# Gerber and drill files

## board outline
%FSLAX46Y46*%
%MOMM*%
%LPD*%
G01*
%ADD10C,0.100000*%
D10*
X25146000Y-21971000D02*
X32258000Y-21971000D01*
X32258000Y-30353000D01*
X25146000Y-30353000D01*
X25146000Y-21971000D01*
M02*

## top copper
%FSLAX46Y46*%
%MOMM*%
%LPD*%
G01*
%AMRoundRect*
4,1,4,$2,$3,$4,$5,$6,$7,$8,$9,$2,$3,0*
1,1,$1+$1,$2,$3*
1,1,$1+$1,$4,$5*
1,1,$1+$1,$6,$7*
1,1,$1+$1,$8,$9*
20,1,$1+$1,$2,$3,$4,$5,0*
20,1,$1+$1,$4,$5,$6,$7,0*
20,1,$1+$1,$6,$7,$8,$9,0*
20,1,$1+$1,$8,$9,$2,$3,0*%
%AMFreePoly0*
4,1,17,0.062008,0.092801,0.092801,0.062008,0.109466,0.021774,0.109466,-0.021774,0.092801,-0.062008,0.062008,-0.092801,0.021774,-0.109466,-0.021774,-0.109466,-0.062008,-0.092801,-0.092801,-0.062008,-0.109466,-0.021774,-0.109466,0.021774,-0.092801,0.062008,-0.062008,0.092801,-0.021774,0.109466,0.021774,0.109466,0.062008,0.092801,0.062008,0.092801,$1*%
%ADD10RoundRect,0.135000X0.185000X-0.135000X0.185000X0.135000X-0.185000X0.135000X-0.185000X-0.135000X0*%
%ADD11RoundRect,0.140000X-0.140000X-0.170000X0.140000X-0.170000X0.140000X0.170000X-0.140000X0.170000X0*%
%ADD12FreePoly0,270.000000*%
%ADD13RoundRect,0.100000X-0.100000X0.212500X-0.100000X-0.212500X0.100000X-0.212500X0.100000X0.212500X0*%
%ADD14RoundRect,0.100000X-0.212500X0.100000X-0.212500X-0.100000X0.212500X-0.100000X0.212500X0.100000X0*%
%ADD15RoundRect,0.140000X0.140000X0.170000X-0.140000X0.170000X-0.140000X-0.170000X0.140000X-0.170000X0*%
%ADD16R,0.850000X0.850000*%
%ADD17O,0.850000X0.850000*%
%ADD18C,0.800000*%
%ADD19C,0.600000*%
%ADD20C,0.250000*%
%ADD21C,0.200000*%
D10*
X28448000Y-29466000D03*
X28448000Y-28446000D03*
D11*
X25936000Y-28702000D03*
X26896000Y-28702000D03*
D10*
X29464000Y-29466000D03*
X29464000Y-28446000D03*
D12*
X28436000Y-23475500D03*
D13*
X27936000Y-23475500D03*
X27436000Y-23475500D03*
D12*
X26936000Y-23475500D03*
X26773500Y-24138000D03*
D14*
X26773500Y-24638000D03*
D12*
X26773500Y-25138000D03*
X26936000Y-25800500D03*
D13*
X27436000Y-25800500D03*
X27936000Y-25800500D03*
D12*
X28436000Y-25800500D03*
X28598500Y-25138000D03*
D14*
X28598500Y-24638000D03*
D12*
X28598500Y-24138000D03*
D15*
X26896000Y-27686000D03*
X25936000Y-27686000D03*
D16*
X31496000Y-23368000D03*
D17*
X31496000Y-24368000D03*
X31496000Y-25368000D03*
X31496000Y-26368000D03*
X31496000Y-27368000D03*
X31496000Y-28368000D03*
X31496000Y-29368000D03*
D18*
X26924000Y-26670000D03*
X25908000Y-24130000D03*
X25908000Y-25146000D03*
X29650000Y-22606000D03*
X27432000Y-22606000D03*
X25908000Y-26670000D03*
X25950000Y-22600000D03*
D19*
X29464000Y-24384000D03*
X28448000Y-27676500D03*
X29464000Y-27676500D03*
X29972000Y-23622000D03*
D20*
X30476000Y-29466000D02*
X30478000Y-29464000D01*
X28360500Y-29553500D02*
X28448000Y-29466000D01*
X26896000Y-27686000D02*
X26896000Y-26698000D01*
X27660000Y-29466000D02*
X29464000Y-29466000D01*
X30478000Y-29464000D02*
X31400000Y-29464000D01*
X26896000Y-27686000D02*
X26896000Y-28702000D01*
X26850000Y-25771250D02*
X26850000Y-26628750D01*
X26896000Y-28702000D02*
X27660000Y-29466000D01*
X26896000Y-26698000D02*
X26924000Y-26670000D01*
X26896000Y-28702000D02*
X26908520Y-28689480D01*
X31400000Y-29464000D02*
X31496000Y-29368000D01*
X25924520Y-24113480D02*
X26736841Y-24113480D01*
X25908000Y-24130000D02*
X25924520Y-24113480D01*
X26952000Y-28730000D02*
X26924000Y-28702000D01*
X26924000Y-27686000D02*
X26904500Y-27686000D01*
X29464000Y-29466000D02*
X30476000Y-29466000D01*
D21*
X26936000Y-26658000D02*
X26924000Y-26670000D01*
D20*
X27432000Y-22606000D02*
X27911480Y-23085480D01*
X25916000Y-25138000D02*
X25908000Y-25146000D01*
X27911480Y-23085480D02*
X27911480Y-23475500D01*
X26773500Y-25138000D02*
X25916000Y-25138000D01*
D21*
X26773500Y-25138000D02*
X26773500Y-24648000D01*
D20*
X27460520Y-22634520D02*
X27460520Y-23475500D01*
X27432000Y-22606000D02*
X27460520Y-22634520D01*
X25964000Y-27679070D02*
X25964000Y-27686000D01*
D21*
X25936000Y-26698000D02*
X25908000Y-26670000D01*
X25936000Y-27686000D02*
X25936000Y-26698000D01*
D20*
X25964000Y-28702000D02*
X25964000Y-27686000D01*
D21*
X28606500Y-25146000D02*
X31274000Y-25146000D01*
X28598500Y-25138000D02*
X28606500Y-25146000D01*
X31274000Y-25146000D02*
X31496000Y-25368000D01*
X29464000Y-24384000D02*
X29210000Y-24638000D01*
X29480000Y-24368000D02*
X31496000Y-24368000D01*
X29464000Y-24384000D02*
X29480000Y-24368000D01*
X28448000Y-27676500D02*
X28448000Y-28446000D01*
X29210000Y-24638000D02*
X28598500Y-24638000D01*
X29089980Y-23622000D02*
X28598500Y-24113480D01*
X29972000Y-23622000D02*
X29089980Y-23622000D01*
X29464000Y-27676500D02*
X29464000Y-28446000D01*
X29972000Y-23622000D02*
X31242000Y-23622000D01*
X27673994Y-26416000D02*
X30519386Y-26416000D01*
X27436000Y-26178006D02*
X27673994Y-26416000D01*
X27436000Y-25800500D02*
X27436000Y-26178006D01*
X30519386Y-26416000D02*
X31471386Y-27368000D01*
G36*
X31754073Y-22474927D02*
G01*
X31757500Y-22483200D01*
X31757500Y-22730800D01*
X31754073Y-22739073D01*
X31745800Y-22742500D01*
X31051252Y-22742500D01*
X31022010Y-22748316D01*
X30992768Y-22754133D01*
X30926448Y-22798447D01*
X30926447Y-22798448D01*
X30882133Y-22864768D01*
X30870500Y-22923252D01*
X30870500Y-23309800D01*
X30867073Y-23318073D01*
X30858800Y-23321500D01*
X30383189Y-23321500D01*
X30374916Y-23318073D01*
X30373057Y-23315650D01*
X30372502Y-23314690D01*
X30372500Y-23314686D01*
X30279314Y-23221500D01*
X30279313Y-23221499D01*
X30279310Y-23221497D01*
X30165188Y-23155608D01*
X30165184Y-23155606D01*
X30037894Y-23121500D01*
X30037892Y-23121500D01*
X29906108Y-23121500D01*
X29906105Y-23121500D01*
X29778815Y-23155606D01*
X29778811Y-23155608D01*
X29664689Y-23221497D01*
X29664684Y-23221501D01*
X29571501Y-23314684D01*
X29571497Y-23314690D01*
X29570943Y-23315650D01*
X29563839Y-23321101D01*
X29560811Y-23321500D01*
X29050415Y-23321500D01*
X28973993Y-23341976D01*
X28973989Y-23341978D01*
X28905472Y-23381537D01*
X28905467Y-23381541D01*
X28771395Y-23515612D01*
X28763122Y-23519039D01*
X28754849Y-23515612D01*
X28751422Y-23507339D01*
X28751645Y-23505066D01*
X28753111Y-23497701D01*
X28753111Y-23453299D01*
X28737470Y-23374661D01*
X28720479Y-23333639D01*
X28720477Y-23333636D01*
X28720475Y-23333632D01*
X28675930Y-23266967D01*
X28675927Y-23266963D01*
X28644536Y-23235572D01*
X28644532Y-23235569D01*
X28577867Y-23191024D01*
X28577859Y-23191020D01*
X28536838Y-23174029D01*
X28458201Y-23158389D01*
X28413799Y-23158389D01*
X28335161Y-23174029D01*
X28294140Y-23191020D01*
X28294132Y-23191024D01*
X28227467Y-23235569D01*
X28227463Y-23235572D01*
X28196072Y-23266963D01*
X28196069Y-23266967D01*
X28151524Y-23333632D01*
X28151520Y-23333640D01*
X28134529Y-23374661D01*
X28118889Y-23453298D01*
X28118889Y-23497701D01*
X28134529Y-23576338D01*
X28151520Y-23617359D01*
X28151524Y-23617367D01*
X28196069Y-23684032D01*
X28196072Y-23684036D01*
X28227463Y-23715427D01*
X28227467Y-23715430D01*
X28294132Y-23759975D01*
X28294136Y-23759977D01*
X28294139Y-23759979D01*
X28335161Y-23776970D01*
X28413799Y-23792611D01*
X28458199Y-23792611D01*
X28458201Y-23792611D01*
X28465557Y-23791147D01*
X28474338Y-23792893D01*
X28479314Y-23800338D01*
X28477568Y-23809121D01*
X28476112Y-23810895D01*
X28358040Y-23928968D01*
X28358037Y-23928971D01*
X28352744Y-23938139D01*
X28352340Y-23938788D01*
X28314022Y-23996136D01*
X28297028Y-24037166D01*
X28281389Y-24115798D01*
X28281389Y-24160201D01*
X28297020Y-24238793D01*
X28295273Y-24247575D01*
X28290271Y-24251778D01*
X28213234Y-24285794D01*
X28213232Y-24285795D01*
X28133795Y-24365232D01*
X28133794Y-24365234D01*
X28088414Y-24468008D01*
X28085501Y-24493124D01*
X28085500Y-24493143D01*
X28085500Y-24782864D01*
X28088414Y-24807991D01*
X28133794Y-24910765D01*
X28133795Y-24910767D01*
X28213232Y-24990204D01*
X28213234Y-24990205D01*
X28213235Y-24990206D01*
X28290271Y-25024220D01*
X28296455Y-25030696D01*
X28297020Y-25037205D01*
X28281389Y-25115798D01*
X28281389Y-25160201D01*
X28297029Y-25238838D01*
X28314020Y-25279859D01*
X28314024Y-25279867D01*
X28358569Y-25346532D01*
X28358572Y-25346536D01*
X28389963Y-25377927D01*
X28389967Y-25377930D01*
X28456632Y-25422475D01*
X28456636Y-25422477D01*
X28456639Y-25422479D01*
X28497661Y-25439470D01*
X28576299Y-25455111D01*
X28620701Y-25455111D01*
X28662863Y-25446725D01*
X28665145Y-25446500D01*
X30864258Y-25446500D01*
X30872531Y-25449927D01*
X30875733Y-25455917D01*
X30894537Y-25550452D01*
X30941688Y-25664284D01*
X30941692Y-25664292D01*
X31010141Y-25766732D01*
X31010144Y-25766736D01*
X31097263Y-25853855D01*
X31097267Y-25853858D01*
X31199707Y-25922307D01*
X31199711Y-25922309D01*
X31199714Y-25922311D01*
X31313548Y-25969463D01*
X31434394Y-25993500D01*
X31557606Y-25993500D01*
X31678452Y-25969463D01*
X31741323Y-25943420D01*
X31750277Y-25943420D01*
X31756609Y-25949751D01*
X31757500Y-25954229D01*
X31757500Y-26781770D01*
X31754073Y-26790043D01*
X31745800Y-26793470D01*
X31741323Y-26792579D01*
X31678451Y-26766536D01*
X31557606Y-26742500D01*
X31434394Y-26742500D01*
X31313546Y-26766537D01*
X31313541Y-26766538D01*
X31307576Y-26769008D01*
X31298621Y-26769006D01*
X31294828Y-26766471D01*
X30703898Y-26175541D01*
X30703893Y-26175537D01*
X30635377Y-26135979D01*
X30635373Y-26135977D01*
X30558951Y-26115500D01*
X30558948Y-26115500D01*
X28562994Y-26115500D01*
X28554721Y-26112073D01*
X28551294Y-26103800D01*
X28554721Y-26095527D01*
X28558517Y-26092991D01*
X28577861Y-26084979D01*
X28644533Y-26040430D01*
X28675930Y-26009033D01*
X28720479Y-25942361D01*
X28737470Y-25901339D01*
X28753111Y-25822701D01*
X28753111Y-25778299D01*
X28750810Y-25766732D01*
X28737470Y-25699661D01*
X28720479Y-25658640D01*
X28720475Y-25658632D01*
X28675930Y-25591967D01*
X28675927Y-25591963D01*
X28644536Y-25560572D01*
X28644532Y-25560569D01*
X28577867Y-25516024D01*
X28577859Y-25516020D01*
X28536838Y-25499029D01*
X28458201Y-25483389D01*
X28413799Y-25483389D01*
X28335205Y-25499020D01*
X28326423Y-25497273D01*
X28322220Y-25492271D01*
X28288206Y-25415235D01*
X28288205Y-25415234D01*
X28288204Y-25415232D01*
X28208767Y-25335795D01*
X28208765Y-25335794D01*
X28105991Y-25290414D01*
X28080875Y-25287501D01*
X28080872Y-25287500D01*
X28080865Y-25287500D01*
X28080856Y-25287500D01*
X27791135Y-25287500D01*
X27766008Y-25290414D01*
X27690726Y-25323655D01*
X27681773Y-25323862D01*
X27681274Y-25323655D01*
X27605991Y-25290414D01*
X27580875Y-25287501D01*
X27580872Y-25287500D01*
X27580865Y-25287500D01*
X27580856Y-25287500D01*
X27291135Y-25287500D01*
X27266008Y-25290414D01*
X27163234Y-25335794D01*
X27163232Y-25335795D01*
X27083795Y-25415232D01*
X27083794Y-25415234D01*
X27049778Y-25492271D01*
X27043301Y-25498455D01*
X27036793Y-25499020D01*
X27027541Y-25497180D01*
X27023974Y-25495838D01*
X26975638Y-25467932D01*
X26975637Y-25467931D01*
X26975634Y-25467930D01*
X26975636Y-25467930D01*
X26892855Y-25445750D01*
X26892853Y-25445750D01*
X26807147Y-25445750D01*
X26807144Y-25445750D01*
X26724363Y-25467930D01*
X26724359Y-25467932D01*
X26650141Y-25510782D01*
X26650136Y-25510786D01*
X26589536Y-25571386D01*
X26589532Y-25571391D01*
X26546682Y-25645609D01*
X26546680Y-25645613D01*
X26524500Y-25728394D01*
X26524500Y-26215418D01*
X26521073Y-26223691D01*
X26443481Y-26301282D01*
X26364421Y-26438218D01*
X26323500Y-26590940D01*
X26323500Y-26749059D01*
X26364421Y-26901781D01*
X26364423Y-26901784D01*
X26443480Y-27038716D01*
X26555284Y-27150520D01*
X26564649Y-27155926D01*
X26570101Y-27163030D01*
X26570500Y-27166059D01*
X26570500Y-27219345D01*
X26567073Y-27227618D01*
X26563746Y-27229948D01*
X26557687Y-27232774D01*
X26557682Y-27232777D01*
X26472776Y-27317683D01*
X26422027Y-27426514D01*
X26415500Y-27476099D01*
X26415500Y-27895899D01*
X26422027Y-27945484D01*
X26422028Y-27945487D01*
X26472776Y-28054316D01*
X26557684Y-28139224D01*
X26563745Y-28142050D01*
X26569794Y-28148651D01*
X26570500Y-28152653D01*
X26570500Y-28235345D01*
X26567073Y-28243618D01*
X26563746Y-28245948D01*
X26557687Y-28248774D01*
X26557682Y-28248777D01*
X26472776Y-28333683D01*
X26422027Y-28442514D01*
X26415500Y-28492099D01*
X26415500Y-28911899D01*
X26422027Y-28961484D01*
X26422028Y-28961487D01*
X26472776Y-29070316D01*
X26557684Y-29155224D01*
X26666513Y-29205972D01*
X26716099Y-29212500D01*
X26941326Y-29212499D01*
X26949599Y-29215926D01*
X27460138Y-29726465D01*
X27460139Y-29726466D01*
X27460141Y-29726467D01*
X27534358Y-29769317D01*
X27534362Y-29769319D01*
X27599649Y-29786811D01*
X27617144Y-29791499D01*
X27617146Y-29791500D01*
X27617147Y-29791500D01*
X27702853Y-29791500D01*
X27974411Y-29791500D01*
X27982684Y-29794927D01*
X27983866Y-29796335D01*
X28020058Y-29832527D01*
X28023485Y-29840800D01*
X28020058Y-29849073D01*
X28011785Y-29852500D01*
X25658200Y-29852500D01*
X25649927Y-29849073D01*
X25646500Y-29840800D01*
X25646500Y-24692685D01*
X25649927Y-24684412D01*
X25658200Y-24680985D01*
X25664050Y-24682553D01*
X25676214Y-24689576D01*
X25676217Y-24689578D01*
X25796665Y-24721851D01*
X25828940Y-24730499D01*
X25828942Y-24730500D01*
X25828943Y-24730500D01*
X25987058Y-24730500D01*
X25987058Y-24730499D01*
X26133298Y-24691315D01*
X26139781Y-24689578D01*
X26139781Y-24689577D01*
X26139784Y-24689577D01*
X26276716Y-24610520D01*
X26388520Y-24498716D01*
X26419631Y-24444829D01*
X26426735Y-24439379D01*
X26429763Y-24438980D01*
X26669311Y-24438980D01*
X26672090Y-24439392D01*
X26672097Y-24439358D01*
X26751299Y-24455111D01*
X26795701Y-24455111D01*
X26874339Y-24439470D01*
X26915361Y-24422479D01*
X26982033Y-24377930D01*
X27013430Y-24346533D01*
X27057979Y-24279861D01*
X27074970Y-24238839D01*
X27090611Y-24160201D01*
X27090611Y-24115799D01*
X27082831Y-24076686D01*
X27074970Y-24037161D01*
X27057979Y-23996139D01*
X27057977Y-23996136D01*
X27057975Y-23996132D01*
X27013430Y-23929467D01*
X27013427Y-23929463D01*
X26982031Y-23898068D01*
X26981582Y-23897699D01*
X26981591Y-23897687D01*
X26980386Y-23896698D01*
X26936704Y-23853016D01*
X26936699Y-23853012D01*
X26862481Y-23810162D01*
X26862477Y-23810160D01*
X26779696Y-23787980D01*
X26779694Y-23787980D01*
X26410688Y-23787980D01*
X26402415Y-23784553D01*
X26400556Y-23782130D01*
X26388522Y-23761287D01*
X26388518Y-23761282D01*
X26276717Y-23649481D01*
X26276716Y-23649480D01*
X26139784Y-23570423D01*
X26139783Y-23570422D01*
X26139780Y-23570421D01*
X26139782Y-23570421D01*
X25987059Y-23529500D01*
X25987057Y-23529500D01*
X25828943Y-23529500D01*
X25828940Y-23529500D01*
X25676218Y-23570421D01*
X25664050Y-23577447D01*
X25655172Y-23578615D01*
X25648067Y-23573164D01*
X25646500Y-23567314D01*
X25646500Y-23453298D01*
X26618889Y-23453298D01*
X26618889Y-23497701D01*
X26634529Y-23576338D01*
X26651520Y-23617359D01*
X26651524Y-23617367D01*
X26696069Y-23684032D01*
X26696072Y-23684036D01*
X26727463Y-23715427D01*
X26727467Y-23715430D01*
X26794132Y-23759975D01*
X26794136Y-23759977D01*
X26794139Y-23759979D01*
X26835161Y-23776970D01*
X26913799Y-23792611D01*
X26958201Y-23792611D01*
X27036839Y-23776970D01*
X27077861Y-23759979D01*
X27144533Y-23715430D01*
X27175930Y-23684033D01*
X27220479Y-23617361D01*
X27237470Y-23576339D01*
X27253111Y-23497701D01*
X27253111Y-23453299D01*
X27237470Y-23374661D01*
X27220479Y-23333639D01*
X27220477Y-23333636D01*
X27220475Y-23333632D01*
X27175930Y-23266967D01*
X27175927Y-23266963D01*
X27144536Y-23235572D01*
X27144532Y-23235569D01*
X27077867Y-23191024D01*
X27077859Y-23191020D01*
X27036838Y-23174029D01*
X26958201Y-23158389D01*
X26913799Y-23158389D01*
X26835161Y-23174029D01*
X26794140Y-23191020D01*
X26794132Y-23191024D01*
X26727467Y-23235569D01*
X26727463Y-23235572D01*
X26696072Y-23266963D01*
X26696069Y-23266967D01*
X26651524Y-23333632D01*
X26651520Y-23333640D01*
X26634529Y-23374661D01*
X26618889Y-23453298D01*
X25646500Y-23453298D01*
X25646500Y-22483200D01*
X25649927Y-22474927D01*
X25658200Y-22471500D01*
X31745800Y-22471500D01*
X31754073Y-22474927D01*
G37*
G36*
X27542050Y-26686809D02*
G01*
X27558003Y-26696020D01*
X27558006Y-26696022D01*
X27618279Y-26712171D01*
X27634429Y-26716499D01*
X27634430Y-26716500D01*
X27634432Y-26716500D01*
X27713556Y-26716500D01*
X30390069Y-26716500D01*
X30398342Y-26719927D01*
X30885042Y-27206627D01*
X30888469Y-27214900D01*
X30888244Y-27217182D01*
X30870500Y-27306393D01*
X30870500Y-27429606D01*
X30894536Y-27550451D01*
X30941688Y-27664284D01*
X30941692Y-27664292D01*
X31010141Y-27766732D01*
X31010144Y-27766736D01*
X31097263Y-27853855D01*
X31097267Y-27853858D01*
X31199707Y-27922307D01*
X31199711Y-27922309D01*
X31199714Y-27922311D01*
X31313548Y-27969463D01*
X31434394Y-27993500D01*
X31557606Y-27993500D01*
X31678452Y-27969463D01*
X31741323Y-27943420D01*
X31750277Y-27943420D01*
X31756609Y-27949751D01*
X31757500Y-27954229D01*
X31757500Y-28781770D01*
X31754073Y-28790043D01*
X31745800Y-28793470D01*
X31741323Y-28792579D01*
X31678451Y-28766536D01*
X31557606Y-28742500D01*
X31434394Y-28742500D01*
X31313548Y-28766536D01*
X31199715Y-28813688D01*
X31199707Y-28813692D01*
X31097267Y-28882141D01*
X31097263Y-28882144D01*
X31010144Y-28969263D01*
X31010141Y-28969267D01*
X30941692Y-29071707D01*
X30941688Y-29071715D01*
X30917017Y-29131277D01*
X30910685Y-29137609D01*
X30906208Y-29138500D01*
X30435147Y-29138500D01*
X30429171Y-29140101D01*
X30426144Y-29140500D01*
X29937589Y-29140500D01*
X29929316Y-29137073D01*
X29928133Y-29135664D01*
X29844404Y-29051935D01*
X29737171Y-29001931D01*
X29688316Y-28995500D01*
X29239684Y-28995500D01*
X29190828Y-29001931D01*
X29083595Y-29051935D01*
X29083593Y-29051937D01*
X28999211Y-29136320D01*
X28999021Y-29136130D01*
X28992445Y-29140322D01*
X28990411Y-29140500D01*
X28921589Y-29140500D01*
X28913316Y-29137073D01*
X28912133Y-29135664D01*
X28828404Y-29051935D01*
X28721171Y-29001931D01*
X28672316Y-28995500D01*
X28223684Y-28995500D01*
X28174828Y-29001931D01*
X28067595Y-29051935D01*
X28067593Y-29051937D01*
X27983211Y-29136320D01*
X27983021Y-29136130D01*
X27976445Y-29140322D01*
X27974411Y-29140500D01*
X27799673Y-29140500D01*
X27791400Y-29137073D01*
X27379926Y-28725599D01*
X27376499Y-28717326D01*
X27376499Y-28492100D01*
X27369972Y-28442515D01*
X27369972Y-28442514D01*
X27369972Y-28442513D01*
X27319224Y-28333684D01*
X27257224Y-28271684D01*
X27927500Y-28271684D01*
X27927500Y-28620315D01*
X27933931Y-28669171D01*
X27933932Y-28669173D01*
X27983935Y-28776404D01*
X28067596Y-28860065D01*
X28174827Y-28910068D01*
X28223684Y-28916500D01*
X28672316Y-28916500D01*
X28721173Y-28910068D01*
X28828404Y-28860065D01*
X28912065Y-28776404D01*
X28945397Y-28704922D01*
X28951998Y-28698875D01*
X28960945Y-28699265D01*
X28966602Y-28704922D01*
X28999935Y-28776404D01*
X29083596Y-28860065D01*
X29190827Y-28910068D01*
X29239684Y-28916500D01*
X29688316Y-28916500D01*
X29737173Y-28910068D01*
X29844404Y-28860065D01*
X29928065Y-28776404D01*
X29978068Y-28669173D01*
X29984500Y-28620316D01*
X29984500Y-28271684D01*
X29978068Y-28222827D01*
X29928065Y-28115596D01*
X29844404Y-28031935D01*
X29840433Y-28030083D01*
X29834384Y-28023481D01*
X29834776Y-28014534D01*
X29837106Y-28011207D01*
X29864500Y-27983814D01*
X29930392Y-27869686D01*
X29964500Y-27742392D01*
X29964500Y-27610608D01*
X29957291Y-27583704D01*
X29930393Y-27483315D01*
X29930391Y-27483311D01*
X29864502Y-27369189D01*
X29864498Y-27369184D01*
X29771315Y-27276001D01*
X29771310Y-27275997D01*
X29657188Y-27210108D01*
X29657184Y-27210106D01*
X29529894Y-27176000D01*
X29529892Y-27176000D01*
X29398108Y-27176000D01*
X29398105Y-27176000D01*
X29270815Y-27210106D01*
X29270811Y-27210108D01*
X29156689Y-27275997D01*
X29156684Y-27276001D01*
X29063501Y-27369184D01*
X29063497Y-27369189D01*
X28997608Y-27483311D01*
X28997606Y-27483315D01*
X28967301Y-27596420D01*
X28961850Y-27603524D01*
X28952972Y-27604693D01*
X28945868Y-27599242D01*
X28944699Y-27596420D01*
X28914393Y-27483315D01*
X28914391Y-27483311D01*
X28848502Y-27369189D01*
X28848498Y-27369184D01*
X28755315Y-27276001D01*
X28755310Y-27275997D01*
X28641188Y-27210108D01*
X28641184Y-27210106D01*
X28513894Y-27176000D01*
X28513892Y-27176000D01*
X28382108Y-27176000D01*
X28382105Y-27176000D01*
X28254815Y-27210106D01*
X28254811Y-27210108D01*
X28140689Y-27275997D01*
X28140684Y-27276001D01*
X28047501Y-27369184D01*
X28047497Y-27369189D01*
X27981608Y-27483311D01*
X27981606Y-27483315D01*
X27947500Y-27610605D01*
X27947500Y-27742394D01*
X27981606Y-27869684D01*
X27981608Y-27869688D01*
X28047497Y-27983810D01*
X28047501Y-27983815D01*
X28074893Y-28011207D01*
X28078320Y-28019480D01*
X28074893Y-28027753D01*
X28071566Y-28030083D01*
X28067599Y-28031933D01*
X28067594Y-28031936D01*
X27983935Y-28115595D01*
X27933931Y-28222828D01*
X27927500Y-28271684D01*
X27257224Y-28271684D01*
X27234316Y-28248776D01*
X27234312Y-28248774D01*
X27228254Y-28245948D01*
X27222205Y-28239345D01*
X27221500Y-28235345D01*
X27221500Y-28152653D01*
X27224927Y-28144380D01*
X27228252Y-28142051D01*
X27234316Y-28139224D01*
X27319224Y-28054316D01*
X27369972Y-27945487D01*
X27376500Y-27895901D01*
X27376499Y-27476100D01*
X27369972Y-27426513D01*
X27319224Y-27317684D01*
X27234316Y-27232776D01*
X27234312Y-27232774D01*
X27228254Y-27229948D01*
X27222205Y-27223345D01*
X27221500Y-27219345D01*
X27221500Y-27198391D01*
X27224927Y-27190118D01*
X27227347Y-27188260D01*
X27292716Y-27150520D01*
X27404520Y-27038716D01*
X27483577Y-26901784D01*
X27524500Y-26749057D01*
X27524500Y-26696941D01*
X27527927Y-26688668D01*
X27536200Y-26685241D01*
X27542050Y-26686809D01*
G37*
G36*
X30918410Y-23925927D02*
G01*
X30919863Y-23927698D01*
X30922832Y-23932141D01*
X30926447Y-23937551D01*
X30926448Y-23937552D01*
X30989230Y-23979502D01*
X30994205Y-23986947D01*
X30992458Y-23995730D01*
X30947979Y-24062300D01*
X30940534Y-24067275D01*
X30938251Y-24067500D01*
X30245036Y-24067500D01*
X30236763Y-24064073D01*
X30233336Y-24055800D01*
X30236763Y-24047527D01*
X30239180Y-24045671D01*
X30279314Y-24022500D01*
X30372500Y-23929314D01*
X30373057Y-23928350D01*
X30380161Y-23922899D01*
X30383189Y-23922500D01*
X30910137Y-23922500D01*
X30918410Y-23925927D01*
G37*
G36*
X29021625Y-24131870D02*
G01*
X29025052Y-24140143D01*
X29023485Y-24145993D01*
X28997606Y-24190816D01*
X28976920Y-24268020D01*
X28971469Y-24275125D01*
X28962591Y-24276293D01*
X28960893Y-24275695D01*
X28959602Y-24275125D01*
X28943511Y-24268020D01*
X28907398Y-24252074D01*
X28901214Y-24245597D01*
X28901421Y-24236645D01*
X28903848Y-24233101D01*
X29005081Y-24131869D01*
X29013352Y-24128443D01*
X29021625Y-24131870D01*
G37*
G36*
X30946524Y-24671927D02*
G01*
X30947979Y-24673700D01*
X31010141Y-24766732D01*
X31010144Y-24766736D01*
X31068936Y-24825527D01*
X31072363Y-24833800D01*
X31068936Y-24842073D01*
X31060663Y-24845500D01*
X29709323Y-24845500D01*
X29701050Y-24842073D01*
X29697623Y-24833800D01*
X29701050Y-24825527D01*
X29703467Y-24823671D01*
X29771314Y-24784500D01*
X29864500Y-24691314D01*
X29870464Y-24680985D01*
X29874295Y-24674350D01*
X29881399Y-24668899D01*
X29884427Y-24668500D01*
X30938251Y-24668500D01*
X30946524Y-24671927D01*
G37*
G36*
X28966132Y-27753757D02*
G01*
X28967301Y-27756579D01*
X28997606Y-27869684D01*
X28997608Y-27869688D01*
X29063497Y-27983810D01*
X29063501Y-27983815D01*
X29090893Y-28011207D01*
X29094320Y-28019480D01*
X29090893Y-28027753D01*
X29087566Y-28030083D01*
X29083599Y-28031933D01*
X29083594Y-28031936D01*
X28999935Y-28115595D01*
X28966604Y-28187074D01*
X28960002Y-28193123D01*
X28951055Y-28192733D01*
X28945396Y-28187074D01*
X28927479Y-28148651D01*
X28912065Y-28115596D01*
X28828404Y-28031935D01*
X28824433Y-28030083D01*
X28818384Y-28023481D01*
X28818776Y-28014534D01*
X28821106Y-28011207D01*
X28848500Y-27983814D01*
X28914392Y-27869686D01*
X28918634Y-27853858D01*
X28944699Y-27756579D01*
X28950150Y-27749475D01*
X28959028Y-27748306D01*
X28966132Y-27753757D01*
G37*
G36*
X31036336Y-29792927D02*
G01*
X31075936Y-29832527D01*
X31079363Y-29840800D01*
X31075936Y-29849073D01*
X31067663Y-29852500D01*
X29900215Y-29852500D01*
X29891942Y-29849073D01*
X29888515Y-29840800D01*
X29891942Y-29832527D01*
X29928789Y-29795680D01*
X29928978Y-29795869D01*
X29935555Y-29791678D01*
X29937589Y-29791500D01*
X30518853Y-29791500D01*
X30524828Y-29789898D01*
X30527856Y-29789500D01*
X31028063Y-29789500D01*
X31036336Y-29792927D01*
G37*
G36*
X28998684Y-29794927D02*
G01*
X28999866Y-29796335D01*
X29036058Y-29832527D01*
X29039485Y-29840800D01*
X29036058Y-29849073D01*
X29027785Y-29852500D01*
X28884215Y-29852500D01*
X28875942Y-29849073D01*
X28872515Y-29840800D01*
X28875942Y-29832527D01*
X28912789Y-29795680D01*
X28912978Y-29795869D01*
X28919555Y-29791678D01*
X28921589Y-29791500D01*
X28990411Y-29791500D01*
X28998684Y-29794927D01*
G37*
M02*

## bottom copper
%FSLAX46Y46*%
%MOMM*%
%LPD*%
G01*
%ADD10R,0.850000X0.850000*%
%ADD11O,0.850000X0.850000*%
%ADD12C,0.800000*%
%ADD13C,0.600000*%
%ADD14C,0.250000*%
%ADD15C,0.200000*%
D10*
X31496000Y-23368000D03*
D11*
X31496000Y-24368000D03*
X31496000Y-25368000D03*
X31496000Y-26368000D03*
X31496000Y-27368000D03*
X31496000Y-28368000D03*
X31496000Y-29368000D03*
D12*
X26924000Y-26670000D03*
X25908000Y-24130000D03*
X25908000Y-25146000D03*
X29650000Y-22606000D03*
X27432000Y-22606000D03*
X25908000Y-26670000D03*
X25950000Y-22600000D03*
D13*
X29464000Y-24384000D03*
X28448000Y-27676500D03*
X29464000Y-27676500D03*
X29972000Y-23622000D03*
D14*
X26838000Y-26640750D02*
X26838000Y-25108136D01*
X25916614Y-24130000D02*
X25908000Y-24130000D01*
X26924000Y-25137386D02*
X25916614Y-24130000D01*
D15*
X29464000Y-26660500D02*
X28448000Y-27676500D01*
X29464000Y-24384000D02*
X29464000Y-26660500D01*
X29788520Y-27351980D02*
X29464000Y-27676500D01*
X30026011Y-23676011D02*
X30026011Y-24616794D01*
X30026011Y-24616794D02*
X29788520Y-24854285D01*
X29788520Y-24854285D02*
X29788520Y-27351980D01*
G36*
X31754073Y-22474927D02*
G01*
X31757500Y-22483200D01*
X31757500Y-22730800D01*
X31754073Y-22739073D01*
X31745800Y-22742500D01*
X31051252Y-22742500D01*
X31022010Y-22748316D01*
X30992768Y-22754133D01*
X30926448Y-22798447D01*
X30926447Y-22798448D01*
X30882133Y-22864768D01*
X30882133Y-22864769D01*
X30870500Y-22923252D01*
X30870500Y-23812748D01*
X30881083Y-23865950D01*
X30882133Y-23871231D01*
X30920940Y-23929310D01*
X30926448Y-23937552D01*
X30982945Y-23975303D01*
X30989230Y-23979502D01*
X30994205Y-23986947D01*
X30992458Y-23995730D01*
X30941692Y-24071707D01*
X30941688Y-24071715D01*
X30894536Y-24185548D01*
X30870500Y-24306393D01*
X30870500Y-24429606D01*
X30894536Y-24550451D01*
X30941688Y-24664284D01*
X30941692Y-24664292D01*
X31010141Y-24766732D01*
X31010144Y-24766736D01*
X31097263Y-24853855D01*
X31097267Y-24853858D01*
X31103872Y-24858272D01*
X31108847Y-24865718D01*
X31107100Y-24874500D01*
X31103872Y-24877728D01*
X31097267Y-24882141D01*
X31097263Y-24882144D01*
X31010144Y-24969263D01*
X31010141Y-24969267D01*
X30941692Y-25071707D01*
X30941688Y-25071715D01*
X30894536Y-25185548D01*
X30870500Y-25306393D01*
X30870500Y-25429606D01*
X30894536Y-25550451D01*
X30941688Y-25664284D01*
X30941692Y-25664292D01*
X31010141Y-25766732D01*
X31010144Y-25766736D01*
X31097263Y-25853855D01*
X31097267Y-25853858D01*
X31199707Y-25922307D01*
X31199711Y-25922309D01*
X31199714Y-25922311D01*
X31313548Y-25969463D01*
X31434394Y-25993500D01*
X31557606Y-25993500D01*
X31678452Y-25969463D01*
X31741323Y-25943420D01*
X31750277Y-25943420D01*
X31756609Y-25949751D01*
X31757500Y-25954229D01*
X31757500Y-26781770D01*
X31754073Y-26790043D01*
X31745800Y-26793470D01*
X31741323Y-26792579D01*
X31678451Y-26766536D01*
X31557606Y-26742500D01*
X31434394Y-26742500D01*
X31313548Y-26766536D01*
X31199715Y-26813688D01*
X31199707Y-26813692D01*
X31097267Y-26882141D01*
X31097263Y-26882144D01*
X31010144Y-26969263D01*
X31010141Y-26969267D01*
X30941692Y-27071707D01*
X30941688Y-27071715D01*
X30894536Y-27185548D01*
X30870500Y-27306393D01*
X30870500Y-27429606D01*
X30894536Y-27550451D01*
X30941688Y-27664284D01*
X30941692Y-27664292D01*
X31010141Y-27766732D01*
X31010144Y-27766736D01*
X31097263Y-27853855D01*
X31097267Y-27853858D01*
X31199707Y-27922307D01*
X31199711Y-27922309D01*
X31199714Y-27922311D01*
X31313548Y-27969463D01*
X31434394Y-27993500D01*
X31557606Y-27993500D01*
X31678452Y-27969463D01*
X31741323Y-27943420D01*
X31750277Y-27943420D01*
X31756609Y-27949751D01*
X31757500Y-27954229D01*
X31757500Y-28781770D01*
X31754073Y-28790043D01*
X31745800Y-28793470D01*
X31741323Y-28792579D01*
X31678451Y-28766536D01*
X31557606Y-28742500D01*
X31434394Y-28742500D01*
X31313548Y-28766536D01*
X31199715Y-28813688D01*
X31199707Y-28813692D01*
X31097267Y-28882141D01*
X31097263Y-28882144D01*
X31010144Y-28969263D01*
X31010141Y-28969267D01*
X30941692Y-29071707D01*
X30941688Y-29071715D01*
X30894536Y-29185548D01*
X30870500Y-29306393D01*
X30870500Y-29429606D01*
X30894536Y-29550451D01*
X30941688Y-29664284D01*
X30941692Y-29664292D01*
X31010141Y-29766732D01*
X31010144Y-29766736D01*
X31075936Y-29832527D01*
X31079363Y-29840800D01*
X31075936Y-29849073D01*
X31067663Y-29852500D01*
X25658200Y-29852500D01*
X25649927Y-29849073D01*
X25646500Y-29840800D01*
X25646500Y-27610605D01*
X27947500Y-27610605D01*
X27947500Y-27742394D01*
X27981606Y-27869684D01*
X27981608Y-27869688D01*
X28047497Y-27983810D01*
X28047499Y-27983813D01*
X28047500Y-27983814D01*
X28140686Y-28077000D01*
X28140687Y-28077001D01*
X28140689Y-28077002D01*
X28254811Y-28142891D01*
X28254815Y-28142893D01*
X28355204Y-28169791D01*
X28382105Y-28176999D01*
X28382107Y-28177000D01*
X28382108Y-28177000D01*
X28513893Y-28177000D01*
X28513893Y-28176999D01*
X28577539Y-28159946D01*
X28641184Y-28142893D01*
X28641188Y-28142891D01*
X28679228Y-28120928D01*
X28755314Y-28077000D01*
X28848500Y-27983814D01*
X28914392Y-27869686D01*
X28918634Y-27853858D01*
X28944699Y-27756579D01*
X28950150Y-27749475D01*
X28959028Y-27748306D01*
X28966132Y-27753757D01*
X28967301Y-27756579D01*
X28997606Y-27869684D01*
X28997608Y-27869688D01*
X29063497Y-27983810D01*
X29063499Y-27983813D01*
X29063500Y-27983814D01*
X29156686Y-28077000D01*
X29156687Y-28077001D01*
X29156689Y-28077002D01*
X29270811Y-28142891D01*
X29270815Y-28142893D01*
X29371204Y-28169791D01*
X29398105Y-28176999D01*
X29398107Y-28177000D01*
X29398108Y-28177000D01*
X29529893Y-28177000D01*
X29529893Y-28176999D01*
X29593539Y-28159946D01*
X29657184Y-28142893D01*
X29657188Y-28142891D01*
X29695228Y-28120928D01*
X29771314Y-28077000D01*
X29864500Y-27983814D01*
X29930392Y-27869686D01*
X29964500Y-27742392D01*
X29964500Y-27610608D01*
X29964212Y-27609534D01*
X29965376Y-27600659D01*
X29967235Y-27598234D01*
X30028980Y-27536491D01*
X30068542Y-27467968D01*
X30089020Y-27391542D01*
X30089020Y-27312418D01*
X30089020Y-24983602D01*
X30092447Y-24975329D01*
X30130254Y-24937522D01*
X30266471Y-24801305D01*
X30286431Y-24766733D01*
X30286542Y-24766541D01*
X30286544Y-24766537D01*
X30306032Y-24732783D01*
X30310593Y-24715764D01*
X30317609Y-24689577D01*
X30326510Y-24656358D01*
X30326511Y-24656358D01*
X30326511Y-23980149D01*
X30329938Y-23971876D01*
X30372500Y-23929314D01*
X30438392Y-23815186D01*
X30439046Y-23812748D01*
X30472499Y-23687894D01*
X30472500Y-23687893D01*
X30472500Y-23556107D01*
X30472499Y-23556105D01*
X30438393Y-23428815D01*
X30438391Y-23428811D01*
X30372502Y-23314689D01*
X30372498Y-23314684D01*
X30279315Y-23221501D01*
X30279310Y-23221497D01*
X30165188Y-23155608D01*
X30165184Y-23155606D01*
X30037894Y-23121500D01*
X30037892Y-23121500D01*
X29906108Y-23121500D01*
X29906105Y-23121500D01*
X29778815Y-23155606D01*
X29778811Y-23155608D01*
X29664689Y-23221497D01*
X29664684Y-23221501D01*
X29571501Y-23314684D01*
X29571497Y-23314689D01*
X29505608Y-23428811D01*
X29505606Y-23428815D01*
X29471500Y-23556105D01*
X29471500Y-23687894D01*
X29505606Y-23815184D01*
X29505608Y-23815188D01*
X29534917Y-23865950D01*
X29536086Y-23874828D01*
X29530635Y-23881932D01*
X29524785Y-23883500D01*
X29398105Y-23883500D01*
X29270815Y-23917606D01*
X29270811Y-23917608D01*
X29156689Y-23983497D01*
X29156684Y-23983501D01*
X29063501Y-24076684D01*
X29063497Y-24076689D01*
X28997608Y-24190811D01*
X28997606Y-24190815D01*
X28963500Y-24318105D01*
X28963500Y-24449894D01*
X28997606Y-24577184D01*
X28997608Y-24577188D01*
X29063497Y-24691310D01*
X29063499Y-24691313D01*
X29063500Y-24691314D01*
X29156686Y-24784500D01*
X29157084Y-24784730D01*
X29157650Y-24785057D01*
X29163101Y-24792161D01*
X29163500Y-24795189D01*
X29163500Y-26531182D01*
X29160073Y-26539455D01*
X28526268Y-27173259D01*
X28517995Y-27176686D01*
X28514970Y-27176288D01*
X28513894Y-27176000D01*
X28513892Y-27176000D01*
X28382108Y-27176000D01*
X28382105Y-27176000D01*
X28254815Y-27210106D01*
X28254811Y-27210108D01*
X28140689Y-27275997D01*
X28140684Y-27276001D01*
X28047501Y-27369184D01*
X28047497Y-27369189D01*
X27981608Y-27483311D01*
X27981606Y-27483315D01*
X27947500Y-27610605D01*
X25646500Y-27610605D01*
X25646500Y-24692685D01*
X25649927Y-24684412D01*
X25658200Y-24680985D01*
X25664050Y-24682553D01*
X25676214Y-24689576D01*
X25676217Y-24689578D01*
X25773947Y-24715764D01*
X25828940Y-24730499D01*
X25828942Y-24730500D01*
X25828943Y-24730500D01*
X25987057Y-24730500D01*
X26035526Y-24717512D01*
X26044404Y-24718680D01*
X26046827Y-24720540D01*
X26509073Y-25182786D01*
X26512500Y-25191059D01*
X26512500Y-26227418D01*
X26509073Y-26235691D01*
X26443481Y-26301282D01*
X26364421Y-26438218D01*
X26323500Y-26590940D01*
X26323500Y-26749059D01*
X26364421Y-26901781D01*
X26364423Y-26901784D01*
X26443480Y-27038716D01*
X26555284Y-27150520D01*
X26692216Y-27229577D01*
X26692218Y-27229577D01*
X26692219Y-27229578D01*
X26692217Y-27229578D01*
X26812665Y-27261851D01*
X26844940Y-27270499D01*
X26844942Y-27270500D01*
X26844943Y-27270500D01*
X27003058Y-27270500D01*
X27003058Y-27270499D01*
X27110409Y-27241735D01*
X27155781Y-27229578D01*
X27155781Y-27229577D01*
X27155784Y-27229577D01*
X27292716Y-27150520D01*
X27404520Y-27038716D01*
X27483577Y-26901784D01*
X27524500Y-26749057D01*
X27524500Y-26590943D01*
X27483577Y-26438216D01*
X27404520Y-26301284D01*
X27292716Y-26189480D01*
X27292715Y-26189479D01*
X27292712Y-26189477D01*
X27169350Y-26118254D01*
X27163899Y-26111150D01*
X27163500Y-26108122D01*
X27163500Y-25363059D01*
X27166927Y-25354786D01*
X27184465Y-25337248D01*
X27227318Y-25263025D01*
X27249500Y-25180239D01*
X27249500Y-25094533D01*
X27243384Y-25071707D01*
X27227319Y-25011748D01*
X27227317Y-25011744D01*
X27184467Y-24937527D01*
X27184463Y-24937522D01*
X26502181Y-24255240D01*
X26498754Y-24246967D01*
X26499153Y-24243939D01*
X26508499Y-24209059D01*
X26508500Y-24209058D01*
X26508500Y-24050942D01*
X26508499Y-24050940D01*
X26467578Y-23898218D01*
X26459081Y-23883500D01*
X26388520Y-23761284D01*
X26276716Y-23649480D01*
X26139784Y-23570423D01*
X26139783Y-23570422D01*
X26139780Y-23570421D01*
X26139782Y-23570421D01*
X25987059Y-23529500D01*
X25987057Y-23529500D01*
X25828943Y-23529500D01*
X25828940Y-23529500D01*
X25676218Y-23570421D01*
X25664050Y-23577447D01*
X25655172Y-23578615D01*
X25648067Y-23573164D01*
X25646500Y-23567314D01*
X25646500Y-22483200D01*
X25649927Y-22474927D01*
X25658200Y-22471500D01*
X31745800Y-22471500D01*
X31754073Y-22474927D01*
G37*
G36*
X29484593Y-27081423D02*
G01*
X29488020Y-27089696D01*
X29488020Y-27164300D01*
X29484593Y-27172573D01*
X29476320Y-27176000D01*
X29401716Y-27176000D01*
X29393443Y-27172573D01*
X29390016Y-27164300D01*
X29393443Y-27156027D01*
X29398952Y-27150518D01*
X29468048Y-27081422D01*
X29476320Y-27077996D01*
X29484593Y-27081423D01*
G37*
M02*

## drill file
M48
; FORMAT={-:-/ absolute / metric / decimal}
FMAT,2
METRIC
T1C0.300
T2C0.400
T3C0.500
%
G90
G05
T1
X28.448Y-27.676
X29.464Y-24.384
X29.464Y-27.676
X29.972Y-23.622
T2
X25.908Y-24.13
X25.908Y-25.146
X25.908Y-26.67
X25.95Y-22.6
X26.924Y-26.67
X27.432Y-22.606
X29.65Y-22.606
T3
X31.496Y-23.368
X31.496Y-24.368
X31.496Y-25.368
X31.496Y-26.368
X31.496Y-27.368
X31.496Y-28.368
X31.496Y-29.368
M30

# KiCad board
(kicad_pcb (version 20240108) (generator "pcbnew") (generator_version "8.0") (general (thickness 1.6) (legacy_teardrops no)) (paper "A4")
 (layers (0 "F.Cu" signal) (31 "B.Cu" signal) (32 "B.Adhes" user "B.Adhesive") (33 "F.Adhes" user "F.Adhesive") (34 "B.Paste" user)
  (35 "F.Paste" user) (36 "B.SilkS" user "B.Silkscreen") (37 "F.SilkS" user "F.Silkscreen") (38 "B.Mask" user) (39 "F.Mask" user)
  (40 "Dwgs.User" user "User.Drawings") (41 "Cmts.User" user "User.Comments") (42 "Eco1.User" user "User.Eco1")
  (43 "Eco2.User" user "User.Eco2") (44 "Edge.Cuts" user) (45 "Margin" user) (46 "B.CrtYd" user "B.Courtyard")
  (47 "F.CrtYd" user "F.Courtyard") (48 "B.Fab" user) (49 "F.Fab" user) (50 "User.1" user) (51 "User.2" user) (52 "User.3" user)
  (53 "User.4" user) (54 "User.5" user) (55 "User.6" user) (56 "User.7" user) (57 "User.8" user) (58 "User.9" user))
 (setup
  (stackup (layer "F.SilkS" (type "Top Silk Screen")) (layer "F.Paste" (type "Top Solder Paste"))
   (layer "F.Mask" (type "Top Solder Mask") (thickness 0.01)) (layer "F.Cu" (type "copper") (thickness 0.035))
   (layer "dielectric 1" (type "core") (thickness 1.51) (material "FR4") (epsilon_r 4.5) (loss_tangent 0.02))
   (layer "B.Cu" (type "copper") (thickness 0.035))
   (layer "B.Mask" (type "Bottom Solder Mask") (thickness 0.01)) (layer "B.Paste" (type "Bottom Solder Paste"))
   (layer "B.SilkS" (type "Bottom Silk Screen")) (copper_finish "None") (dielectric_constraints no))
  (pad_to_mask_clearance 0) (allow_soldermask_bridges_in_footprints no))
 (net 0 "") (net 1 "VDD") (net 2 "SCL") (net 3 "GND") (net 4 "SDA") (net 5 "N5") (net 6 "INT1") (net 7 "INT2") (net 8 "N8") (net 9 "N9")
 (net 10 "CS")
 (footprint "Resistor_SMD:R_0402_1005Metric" (layer "F.Cu") (at 28.448 28.956 90)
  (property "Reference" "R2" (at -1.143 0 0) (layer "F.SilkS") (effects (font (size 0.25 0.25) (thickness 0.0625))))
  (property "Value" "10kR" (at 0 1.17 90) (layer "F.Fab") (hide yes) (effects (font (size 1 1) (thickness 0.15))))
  (pad "1" smd roundrect (at -0.51 0 90) (size 0.54 0.64) (layers "F.Cu" "F.Paste" "F.Mask") (roundrect_rratio 0.25) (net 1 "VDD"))
  (pad "2" smd roundrect (at 0.51 0 90) (size 0.54 0.64) (layers "F.Cu" "F.Paste" "F.Mask") (roundrect_rratio 0.25) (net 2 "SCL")))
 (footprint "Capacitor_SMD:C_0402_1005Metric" (layer "F.Cu") (at 26.416 28.702)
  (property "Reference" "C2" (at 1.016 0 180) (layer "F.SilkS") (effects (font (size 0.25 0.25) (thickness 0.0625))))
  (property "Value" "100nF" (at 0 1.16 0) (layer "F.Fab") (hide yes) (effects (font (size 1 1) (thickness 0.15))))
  (pad "1" smd roundrect (at -0.48 0) (size 0.56 0.62) (layers "F.Cu" "F.Paste" "F.Mask") (roundrect_rratio 0.25) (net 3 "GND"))
  (pad "2" smd roundrect (at 0.48 0) (size 0.56 0.62) (layers "F.Cu" "F.Paste" "F.Mask") (roundrect_rratio 0.25) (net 1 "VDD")))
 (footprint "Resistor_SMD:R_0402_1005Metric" (layer "F.Cu") (at 29.464 28.956 90)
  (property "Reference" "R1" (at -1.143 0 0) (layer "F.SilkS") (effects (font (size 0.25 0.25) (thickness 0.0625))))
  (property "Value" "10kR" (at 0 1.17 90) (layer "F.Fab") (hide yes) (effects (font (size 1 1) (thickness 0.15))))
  (pad "1" smd roundrect (at -0.51 0 90) (size 0.54 0.64) (layers "F.Cu" "F.Paste" "F.Mask") (roundrect_rratio 0.25) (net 1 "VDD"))
  (pad "2" smd roundrect (at 0.51 0 90) (size 0.54 0.64) (layers "F.Cu" "F.Paste" "F.Mask") (roundrect_rratio 0.25) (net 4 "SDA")))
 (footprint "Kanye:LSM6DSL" (layer "F.Cu") (at 27.686 24.638 -90)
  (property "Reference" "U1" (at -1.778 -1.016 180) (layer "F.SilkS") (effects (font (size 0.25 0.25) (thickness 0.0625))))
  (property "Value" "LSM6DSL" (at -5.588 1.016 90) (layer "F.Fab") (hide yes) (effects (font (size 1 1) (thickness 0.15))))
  (pad "1" smd custom (at -1.1625 -0.75 270) (size 0.223223 0.223223) (layers "F.Cu" "F.Paste" "F.Mask") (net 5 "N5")
   (thermal_bridge_angle 90) (options (clearance outline) (anchor circle)) (primitives))
  (pad "2" smd roundrect (at -1.1625 -0.25 270) (size 0.625 0.4) (layers "F.Cu" "F.Paste" "F.Mask") (roundrect_rratio 0.25) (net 3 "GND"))
  (pad "3" smd roundrect (at -1.1625 0.25 270) (size 0.625 0.4) (layers "F.Cu" "F.Paste" "F.Mask") (roundrect_rratio 0.25) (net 3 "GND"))
  (pad "4" smd custom (at -1.1625 0.75 270) (size 0.223223 0.223223) (layers "F.Cu" "F.Paste" "F.Mask") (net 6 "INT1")
   (thermal_bridge_angle 90) (options (clearance outline) (anchor circle)) (primitives))
  (pad "5" smd custom (at -0.5 0.9125 270) (size 0.223223 0.223223) (layers "F.Cu" "F.Paste" "F.Mask") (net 1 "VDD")
   (thermal_bridge_angle 90) (options (clearance outline) (anchor circle)) (primitives))
  (pad "6" smd roundrect (at 0 0.9125 270) (size 0.4 0.625) (layers "F.Cu" "F.Paste" "F.Mask") (roundrect_rratio 0.25) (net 3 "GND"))
  (pad "7" smd custom (at 0.5 0.9125 270) (size 0.223223 0.223223) (layers "F.Cu" "F.Paste" "F.Mask") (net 3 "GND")
   (thermal_bridge_angle 90) (options (clearance outline) (anchor circle)) (primitives))
  (pad "8" smd custom (at 1.1625 0.75 270) (size 0.223223 0.223223) (layers "F.Cu" "F.Paste" "F.Mask") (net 1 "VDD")
   (thermal_bridge_angle 90) (options (clearance outline) (anchor circle)) (primitives))
  (pad "9" smd roundrect (at 1.1625 0.25 270) (size 0.625 0.4) (layers "F.Cu" "F.Paste" "F.Mask") (roundrect_rratio 0.25) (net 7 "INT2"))
  (pad "10" smd roundrect (at 1.1625 -0.25 270) (size 0.625 0.4) (layers "F.Cu" "F.Paste" "F.Mask") (roundrect_rratio 0.25) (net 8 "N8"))
  (pad "11" smd custom (at 1.1625 -0.75 270) (size 0.223223 0.223223) (layers "F.Cu" "F.Paste" "F.Mask") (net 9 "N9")
   (thermal_bridge_angle 90) (options (clearance outline) (anchor circle)) (primitives))
  (pad "12" smd custom (at 0.5 -0.9125 270) (size 0.223223 0.223223) (layers "F.Cu" "F.Paste" "F.Mask") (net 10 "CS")
   (thermal_bridge_angle 90) (options (clearance outline) (anchor circle)) (primitives))
  (pad "13" smd roundrect (at 0 -0.9125 270) (size 0.4 0.625) (layers "F.Cu" "F.Paste" "F.Mask") (roundrect_rratio 0.25) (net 2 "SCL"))
  (pad "14" smd custom (at -0.5 -0.9125 270) (size 0.223223 0.223223) (layers "F.Cu" "F.Paste" "F.Mask") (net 4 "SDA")
   (thermal_bridge_angle 90) (options (clearance outline) (anchor circle)) (primitives)))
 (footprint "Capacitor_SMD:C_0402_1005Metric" (layer "F.Cu") (at 26.416 27.686 180)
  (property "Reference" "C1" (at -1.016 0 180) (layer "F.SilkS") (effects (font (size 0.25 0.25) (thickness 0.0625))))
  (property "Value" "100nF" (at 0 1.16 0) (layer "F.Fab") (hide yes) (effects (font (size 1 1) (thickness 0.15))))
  (pad "1" smd roundrect (at -0.48 0 180) (size 0.56 0.62) (layers "F.Cu" "F.Paste" "F.Mask") (roundrect_rratio 0.25) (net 1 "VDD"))
  (pad "2" smd roundrect (at 0.48 0 180) (size 0.56 0.62) (layers "F.Cu" "F.Paste" "F.Mask") (roundrect_rratio 0.25) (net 3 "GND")))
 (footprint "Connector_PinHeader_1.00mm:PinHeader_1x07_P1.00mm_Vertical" (layer "F.Cu") (at 31.496 23.368)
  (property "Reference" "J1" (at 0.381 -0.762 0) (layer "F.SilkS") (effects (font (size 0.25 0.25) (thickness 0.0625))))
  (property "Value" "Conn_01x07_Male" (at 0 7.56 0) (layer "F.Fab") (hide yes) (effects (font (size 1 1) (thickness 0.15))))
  (pad "1" thru_hole rect (at 0 0) (size 0.85 0.85) (drill 0.5) (layers "*.Cu" "*.Mask") (remove_unused_layers no) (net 4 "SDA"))
  (pad "2" thru_hole oval (at 0 1) (size 0.85 0.85) (drill 0.5) (layers "*.Cu" "*.Mask") (remove_unused_layers no) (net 2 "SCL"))
  (pad "3" thru_hole oval (at 0 2) (size 0.85 0.85) (drill 0.5) (layers "*.Cu" "*.Mask") (remove_unused_layers no) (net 10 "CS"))
  (pad "4" thru_hole oval (at 0 3) (size 0.85 0.85) (drill 0.5) (layers "*.Cu" "*.Mask") (remove_unused_layers no) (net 3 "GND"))
  (pad "5" thru_hole oval (at 0 4) (size 0.85 0.85) (drill 0.5) (layers "*.Cu" "*.Mask") (remove_unused_layers no) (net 7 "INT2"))
  (pad "6" thru_hole oval (at 0 5) (size 0.85 0.85) (drill 0.5) (layers "*.Cu" "*.Mask") (remove_unused_layers no) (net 3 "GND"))
  (pad "7" thru_hole oval (at 0 6) (size 0.85 0.85) (drill 0.5) (layers "*.Cu" "*.Mask") (remove_unused_layers no) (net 1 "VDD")))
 (gr_rect (start 25.146 21.971) (end 32.258 30.353) (stroke (width 0.1) (type solid)) (fill none) (layer "Edge.Cuts"))
 (segment (start 30.476 29.466) (end 30.478 29.464) (width 0.25) (layer "F.Cu") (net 1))
 (segment (start 28.3605 29.5535) (end 28.448 29.466) (width 0.25) (layer "F.Cu") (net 1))
 (segment (start 26.896 27.686) (end 26.896 26.698) (width 0.25) (layer "F.Cu") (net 1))
 (segment (start 27.66 29.466) (end 29.464 29.466) (width 0.25) (layer "F.Cu") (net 1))
 (segment (start 30.478 29.464) (end 31.4 29.464) (width 0.25) (layer "F.Cu") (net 1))
 (segment (start 26.896 27.686) (end 26.896 28.702) (width 0.25) (layer "F.Cu") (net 1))
 (segment (start 26.85 25.77125) (end 26.85 26.62875) (width 0.25) (layer "F.Cu") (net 1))
 (segment (start 26.896 28.702) (end 27.66 29.466) (width 0.25) (layer "F.Cu") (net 1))
 (segment (start 26.896 26.698) (end 26.924 26.67) (width 0.25) (layer "F.Cu") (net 1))
 (segment (start 26.896 28.702) (end 26.90852 28.68948) (width 0.25) (layer "F.Cu") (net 1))
 (segment (start 31.4 29.464) (end 31.496 29.368) (width 0.25) (layer "F.Cu") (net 1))
 (segment (start 25.92452 24.11348) (end 26.736841 24.11348) (width 0.25) (layer "F.Cu") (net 1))
 (segment (start 25.908 24.13) (end 25.92452 24.11348) (width 0.25) (layer "F.Cu") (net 1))
 (segment (start 26.952 28.73) (end 26.924 28.702) (width 0.25) (layer "F.Cu") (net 1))
 (segment (start 26.924 27.686) (end 26.9045 27.686) (width 0.25) (layer "F.Cu") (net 1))
 (segment (start 29.464 29.466) (end 30.476 29.466) (width 0.25) (layer "F.Cu") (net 1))
 (segment (start 26.936 26.658) (end 26.924 26.67) (width 0.2) (layer "F.Cu") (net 1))
 (via (at 26.924 26.67) (size 0.8) (drill 0.4) (layers "F.Cu" "B.Cu") (free yes) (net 1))
 (via (at 25.908 24.13) (size 0.8) (drill 0.4) (layers "F.Cu" "B.Cu") (free yes) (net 1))
 (segment (start 26.838 26.64075) (end 26.838 25.108136) (width 0.25) (layer "B.Cu") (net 1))
 (segment (start 25.916614 24.13) (end 25.908 24.13) (width 0.25) (layer "B.Cu") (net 1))
 (segment (start 26.924 25.137386) (end 25.916614 24.13) (width 0.25) (layer "B.Cu") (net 1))
 (segment (start 27.432 22.606) (end 27.91148 23.08548) (width 0.25) (layer "F.Cu") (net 3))
 (segment (start 25.916 25.138) (end 25.908 25.146) (width 0.25) (layer "F.Cu") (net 3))
 (segment (start 27.91148 23.08548) (end 27.91148 23.4755) (width 0.25) (layer "F.Cu") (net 3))
 (segment (start 26.7735 25.138) (end 25.916 25.138) (width 0.25) (layer "F.Cu") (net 3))
 (segment (start 26.7735 25.138) (end 26.7735 24.648) (width 0.2) (layer "F.Cu") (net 3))
 (segment (start 27.46052 22.63452) (end 27.46052 23.4755) (width 0.25) (layer "F.Cu") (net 3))
 (segment (start 27.432 22.606) (end 27.46052 22.63452) (width 0.25) (layer "F.Cu") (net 3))
 (segment (start 25.964 27.67907) (end 25.964 27.686) (width 0.25) (layer "F.Cu") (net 3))
 (segment (start 25.936 26.698) (end 25.908 26.67) (width 0.2) (layer "F.Cu") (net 3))
 (segment (start 25.936 27.686) (end 25.936 26.698) (width 0.2) (layer "F.Cu") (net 3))
 (segment (start 25.964 28.702) (end 25.964 27.686) (width 0.25) (layer "F.Cu") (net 3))
 (via (at 25.908 25.146) (size 0.8) (drill 0.4) (layers "F.Cu" "B.Cu") (free yes) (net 3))
 (via (at 29.65 22.606) (size 0.8) (drill 0.4) (layers "F.Cu" "B.Cu") (free yes) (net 3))
 (via (at 27.432 22.606) (size 0.8) (drill 0.4) (layers "F.Cu" "B.Cu") (free yes) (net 3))
 (via (at 25.908 26.67) (size 0.8) (drill 0.4) (layers "F.Cu" "B.Cu") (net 3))
 (via (at 25.95 22.6) (size 0.8) (drill 0.4) (layers "F.Cu" "B.Cu") (free yes) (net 3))
 (segment (start 28.6065 25.146) (end 31.274 25.146) (width 0.2) (layer "F.Cu") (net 10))
 (segment (start 28.5985 25.138) (end 28.6065 25.146) (width 0.2) (layer "F.Cu") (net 10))
 (segment (start 31.274 25.146) (end 31.496 25.368) (width 0.2) (layer "F.Cu") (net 10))
 (segment (start 29.464 24.384) (end 29.21 24.638) (width 0.2) (layer "F.Cu") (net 2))
 (segment (start 29.48 24.368) (end 31.496 24.368) (width 0.2) (layer "F.Cu") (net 2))
 (segment (start 29.464 24.384) (end 29.48 24.368) (width 0.2) (layer "F.Cu") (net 2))
 (segment (start 28.448 27.6765) (end 28.448 28.446) (width 0.2) (layer "F.Cu") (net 2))
 (segment (start 29.21 24.638) (end 28.5985 24.638) (width 0.2) (layer "F.Cu") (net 2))
 (via (at 29.464 24.384) (size 0.6) (drill 0.3) (layers "F.Cu" "B.Cu") (free yes) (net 2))
 (via (at 28.448 27.6765) (size 0.6) (drill 0.3) (layers "F.Cu" "B.Cu") (free yes) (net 2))
 (segment (start 29.464 26.6605) (end 28.448 27.6765) (width 0.2) (layer "B.Cu") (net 2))
 (segment (start 29.464 24.384) (end 29.464 26.6605) (width 0.2) (layer "B.Cu") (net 2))
 (segment (start 29.08998 23.622) (end 28.5985 24.11348) (width 0.2) (layer "F.Cu") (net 4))
 (segment (start 29.972 23.622) (end 29.08998 23.622) (width 0.2) (layer "F.Cu") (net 4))
 (segment (start 29.464 27.6765) (end 29.464 28.446) (width 0.2) (layer "F.Cu") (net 4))
 (segment (start 29.972 23.622) (end 31.242 23.622) (width 0.2) (layer "F.Cu") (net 4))
 (via (at 29.464 27.6765) (size 0.6) (drill 0.3) (layers "F.Cu" "B.Cu") (free yes) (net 4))
 (via (at 29.972 23.622) (size 0.6) (drill 0.3) (layers "F.Cu" "B.Cu") (free yes) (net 4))
 (segment (start 29.78852 27.35198) (end 29.464 27.6765) (width 0.2) (layer "B.Cu") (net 4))
 (segment (start 30.026011 23.676011) (end 30.026011 24.616794) (width 0.2) (layer "B.Cu") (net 4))
 (segment (start 30.026011 24.616794) (end 29.78852 24.854285) (width 0.2) (layer "B.Cu") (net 4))
 (segment (start 29.78852 24.854285) (end 29.78852 27.35198) (width 0.2) (layer "B.Cu") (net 4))
 (segment (start 27.673994 26.416) (end 30.519386 26.416) (width 0.2) (layer "F.Cu") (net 7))
 (segment (start 27.436 26.178006) (end 27.673994 26.416) (width 0.2) (layer "F.Cu") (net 7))
 (segment (start 27.436 25.8005) (end 27.436 26.178006) (width 0.2) (layer "F.Cu") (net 7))
 (segment (start 30.519386 26.416) (end 31.471386 27.368) (width 0.2) (layer "F.Cu") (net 7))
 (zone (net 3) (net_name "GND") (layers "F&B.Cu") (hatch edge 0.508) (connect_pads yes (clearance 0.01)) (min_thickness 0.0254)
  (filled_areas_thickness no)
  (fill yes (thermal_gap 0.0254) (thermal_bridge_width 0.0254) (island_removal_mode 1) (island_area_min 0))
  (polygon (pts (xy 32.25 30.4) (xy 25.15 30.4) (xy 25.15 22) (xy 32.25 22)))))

